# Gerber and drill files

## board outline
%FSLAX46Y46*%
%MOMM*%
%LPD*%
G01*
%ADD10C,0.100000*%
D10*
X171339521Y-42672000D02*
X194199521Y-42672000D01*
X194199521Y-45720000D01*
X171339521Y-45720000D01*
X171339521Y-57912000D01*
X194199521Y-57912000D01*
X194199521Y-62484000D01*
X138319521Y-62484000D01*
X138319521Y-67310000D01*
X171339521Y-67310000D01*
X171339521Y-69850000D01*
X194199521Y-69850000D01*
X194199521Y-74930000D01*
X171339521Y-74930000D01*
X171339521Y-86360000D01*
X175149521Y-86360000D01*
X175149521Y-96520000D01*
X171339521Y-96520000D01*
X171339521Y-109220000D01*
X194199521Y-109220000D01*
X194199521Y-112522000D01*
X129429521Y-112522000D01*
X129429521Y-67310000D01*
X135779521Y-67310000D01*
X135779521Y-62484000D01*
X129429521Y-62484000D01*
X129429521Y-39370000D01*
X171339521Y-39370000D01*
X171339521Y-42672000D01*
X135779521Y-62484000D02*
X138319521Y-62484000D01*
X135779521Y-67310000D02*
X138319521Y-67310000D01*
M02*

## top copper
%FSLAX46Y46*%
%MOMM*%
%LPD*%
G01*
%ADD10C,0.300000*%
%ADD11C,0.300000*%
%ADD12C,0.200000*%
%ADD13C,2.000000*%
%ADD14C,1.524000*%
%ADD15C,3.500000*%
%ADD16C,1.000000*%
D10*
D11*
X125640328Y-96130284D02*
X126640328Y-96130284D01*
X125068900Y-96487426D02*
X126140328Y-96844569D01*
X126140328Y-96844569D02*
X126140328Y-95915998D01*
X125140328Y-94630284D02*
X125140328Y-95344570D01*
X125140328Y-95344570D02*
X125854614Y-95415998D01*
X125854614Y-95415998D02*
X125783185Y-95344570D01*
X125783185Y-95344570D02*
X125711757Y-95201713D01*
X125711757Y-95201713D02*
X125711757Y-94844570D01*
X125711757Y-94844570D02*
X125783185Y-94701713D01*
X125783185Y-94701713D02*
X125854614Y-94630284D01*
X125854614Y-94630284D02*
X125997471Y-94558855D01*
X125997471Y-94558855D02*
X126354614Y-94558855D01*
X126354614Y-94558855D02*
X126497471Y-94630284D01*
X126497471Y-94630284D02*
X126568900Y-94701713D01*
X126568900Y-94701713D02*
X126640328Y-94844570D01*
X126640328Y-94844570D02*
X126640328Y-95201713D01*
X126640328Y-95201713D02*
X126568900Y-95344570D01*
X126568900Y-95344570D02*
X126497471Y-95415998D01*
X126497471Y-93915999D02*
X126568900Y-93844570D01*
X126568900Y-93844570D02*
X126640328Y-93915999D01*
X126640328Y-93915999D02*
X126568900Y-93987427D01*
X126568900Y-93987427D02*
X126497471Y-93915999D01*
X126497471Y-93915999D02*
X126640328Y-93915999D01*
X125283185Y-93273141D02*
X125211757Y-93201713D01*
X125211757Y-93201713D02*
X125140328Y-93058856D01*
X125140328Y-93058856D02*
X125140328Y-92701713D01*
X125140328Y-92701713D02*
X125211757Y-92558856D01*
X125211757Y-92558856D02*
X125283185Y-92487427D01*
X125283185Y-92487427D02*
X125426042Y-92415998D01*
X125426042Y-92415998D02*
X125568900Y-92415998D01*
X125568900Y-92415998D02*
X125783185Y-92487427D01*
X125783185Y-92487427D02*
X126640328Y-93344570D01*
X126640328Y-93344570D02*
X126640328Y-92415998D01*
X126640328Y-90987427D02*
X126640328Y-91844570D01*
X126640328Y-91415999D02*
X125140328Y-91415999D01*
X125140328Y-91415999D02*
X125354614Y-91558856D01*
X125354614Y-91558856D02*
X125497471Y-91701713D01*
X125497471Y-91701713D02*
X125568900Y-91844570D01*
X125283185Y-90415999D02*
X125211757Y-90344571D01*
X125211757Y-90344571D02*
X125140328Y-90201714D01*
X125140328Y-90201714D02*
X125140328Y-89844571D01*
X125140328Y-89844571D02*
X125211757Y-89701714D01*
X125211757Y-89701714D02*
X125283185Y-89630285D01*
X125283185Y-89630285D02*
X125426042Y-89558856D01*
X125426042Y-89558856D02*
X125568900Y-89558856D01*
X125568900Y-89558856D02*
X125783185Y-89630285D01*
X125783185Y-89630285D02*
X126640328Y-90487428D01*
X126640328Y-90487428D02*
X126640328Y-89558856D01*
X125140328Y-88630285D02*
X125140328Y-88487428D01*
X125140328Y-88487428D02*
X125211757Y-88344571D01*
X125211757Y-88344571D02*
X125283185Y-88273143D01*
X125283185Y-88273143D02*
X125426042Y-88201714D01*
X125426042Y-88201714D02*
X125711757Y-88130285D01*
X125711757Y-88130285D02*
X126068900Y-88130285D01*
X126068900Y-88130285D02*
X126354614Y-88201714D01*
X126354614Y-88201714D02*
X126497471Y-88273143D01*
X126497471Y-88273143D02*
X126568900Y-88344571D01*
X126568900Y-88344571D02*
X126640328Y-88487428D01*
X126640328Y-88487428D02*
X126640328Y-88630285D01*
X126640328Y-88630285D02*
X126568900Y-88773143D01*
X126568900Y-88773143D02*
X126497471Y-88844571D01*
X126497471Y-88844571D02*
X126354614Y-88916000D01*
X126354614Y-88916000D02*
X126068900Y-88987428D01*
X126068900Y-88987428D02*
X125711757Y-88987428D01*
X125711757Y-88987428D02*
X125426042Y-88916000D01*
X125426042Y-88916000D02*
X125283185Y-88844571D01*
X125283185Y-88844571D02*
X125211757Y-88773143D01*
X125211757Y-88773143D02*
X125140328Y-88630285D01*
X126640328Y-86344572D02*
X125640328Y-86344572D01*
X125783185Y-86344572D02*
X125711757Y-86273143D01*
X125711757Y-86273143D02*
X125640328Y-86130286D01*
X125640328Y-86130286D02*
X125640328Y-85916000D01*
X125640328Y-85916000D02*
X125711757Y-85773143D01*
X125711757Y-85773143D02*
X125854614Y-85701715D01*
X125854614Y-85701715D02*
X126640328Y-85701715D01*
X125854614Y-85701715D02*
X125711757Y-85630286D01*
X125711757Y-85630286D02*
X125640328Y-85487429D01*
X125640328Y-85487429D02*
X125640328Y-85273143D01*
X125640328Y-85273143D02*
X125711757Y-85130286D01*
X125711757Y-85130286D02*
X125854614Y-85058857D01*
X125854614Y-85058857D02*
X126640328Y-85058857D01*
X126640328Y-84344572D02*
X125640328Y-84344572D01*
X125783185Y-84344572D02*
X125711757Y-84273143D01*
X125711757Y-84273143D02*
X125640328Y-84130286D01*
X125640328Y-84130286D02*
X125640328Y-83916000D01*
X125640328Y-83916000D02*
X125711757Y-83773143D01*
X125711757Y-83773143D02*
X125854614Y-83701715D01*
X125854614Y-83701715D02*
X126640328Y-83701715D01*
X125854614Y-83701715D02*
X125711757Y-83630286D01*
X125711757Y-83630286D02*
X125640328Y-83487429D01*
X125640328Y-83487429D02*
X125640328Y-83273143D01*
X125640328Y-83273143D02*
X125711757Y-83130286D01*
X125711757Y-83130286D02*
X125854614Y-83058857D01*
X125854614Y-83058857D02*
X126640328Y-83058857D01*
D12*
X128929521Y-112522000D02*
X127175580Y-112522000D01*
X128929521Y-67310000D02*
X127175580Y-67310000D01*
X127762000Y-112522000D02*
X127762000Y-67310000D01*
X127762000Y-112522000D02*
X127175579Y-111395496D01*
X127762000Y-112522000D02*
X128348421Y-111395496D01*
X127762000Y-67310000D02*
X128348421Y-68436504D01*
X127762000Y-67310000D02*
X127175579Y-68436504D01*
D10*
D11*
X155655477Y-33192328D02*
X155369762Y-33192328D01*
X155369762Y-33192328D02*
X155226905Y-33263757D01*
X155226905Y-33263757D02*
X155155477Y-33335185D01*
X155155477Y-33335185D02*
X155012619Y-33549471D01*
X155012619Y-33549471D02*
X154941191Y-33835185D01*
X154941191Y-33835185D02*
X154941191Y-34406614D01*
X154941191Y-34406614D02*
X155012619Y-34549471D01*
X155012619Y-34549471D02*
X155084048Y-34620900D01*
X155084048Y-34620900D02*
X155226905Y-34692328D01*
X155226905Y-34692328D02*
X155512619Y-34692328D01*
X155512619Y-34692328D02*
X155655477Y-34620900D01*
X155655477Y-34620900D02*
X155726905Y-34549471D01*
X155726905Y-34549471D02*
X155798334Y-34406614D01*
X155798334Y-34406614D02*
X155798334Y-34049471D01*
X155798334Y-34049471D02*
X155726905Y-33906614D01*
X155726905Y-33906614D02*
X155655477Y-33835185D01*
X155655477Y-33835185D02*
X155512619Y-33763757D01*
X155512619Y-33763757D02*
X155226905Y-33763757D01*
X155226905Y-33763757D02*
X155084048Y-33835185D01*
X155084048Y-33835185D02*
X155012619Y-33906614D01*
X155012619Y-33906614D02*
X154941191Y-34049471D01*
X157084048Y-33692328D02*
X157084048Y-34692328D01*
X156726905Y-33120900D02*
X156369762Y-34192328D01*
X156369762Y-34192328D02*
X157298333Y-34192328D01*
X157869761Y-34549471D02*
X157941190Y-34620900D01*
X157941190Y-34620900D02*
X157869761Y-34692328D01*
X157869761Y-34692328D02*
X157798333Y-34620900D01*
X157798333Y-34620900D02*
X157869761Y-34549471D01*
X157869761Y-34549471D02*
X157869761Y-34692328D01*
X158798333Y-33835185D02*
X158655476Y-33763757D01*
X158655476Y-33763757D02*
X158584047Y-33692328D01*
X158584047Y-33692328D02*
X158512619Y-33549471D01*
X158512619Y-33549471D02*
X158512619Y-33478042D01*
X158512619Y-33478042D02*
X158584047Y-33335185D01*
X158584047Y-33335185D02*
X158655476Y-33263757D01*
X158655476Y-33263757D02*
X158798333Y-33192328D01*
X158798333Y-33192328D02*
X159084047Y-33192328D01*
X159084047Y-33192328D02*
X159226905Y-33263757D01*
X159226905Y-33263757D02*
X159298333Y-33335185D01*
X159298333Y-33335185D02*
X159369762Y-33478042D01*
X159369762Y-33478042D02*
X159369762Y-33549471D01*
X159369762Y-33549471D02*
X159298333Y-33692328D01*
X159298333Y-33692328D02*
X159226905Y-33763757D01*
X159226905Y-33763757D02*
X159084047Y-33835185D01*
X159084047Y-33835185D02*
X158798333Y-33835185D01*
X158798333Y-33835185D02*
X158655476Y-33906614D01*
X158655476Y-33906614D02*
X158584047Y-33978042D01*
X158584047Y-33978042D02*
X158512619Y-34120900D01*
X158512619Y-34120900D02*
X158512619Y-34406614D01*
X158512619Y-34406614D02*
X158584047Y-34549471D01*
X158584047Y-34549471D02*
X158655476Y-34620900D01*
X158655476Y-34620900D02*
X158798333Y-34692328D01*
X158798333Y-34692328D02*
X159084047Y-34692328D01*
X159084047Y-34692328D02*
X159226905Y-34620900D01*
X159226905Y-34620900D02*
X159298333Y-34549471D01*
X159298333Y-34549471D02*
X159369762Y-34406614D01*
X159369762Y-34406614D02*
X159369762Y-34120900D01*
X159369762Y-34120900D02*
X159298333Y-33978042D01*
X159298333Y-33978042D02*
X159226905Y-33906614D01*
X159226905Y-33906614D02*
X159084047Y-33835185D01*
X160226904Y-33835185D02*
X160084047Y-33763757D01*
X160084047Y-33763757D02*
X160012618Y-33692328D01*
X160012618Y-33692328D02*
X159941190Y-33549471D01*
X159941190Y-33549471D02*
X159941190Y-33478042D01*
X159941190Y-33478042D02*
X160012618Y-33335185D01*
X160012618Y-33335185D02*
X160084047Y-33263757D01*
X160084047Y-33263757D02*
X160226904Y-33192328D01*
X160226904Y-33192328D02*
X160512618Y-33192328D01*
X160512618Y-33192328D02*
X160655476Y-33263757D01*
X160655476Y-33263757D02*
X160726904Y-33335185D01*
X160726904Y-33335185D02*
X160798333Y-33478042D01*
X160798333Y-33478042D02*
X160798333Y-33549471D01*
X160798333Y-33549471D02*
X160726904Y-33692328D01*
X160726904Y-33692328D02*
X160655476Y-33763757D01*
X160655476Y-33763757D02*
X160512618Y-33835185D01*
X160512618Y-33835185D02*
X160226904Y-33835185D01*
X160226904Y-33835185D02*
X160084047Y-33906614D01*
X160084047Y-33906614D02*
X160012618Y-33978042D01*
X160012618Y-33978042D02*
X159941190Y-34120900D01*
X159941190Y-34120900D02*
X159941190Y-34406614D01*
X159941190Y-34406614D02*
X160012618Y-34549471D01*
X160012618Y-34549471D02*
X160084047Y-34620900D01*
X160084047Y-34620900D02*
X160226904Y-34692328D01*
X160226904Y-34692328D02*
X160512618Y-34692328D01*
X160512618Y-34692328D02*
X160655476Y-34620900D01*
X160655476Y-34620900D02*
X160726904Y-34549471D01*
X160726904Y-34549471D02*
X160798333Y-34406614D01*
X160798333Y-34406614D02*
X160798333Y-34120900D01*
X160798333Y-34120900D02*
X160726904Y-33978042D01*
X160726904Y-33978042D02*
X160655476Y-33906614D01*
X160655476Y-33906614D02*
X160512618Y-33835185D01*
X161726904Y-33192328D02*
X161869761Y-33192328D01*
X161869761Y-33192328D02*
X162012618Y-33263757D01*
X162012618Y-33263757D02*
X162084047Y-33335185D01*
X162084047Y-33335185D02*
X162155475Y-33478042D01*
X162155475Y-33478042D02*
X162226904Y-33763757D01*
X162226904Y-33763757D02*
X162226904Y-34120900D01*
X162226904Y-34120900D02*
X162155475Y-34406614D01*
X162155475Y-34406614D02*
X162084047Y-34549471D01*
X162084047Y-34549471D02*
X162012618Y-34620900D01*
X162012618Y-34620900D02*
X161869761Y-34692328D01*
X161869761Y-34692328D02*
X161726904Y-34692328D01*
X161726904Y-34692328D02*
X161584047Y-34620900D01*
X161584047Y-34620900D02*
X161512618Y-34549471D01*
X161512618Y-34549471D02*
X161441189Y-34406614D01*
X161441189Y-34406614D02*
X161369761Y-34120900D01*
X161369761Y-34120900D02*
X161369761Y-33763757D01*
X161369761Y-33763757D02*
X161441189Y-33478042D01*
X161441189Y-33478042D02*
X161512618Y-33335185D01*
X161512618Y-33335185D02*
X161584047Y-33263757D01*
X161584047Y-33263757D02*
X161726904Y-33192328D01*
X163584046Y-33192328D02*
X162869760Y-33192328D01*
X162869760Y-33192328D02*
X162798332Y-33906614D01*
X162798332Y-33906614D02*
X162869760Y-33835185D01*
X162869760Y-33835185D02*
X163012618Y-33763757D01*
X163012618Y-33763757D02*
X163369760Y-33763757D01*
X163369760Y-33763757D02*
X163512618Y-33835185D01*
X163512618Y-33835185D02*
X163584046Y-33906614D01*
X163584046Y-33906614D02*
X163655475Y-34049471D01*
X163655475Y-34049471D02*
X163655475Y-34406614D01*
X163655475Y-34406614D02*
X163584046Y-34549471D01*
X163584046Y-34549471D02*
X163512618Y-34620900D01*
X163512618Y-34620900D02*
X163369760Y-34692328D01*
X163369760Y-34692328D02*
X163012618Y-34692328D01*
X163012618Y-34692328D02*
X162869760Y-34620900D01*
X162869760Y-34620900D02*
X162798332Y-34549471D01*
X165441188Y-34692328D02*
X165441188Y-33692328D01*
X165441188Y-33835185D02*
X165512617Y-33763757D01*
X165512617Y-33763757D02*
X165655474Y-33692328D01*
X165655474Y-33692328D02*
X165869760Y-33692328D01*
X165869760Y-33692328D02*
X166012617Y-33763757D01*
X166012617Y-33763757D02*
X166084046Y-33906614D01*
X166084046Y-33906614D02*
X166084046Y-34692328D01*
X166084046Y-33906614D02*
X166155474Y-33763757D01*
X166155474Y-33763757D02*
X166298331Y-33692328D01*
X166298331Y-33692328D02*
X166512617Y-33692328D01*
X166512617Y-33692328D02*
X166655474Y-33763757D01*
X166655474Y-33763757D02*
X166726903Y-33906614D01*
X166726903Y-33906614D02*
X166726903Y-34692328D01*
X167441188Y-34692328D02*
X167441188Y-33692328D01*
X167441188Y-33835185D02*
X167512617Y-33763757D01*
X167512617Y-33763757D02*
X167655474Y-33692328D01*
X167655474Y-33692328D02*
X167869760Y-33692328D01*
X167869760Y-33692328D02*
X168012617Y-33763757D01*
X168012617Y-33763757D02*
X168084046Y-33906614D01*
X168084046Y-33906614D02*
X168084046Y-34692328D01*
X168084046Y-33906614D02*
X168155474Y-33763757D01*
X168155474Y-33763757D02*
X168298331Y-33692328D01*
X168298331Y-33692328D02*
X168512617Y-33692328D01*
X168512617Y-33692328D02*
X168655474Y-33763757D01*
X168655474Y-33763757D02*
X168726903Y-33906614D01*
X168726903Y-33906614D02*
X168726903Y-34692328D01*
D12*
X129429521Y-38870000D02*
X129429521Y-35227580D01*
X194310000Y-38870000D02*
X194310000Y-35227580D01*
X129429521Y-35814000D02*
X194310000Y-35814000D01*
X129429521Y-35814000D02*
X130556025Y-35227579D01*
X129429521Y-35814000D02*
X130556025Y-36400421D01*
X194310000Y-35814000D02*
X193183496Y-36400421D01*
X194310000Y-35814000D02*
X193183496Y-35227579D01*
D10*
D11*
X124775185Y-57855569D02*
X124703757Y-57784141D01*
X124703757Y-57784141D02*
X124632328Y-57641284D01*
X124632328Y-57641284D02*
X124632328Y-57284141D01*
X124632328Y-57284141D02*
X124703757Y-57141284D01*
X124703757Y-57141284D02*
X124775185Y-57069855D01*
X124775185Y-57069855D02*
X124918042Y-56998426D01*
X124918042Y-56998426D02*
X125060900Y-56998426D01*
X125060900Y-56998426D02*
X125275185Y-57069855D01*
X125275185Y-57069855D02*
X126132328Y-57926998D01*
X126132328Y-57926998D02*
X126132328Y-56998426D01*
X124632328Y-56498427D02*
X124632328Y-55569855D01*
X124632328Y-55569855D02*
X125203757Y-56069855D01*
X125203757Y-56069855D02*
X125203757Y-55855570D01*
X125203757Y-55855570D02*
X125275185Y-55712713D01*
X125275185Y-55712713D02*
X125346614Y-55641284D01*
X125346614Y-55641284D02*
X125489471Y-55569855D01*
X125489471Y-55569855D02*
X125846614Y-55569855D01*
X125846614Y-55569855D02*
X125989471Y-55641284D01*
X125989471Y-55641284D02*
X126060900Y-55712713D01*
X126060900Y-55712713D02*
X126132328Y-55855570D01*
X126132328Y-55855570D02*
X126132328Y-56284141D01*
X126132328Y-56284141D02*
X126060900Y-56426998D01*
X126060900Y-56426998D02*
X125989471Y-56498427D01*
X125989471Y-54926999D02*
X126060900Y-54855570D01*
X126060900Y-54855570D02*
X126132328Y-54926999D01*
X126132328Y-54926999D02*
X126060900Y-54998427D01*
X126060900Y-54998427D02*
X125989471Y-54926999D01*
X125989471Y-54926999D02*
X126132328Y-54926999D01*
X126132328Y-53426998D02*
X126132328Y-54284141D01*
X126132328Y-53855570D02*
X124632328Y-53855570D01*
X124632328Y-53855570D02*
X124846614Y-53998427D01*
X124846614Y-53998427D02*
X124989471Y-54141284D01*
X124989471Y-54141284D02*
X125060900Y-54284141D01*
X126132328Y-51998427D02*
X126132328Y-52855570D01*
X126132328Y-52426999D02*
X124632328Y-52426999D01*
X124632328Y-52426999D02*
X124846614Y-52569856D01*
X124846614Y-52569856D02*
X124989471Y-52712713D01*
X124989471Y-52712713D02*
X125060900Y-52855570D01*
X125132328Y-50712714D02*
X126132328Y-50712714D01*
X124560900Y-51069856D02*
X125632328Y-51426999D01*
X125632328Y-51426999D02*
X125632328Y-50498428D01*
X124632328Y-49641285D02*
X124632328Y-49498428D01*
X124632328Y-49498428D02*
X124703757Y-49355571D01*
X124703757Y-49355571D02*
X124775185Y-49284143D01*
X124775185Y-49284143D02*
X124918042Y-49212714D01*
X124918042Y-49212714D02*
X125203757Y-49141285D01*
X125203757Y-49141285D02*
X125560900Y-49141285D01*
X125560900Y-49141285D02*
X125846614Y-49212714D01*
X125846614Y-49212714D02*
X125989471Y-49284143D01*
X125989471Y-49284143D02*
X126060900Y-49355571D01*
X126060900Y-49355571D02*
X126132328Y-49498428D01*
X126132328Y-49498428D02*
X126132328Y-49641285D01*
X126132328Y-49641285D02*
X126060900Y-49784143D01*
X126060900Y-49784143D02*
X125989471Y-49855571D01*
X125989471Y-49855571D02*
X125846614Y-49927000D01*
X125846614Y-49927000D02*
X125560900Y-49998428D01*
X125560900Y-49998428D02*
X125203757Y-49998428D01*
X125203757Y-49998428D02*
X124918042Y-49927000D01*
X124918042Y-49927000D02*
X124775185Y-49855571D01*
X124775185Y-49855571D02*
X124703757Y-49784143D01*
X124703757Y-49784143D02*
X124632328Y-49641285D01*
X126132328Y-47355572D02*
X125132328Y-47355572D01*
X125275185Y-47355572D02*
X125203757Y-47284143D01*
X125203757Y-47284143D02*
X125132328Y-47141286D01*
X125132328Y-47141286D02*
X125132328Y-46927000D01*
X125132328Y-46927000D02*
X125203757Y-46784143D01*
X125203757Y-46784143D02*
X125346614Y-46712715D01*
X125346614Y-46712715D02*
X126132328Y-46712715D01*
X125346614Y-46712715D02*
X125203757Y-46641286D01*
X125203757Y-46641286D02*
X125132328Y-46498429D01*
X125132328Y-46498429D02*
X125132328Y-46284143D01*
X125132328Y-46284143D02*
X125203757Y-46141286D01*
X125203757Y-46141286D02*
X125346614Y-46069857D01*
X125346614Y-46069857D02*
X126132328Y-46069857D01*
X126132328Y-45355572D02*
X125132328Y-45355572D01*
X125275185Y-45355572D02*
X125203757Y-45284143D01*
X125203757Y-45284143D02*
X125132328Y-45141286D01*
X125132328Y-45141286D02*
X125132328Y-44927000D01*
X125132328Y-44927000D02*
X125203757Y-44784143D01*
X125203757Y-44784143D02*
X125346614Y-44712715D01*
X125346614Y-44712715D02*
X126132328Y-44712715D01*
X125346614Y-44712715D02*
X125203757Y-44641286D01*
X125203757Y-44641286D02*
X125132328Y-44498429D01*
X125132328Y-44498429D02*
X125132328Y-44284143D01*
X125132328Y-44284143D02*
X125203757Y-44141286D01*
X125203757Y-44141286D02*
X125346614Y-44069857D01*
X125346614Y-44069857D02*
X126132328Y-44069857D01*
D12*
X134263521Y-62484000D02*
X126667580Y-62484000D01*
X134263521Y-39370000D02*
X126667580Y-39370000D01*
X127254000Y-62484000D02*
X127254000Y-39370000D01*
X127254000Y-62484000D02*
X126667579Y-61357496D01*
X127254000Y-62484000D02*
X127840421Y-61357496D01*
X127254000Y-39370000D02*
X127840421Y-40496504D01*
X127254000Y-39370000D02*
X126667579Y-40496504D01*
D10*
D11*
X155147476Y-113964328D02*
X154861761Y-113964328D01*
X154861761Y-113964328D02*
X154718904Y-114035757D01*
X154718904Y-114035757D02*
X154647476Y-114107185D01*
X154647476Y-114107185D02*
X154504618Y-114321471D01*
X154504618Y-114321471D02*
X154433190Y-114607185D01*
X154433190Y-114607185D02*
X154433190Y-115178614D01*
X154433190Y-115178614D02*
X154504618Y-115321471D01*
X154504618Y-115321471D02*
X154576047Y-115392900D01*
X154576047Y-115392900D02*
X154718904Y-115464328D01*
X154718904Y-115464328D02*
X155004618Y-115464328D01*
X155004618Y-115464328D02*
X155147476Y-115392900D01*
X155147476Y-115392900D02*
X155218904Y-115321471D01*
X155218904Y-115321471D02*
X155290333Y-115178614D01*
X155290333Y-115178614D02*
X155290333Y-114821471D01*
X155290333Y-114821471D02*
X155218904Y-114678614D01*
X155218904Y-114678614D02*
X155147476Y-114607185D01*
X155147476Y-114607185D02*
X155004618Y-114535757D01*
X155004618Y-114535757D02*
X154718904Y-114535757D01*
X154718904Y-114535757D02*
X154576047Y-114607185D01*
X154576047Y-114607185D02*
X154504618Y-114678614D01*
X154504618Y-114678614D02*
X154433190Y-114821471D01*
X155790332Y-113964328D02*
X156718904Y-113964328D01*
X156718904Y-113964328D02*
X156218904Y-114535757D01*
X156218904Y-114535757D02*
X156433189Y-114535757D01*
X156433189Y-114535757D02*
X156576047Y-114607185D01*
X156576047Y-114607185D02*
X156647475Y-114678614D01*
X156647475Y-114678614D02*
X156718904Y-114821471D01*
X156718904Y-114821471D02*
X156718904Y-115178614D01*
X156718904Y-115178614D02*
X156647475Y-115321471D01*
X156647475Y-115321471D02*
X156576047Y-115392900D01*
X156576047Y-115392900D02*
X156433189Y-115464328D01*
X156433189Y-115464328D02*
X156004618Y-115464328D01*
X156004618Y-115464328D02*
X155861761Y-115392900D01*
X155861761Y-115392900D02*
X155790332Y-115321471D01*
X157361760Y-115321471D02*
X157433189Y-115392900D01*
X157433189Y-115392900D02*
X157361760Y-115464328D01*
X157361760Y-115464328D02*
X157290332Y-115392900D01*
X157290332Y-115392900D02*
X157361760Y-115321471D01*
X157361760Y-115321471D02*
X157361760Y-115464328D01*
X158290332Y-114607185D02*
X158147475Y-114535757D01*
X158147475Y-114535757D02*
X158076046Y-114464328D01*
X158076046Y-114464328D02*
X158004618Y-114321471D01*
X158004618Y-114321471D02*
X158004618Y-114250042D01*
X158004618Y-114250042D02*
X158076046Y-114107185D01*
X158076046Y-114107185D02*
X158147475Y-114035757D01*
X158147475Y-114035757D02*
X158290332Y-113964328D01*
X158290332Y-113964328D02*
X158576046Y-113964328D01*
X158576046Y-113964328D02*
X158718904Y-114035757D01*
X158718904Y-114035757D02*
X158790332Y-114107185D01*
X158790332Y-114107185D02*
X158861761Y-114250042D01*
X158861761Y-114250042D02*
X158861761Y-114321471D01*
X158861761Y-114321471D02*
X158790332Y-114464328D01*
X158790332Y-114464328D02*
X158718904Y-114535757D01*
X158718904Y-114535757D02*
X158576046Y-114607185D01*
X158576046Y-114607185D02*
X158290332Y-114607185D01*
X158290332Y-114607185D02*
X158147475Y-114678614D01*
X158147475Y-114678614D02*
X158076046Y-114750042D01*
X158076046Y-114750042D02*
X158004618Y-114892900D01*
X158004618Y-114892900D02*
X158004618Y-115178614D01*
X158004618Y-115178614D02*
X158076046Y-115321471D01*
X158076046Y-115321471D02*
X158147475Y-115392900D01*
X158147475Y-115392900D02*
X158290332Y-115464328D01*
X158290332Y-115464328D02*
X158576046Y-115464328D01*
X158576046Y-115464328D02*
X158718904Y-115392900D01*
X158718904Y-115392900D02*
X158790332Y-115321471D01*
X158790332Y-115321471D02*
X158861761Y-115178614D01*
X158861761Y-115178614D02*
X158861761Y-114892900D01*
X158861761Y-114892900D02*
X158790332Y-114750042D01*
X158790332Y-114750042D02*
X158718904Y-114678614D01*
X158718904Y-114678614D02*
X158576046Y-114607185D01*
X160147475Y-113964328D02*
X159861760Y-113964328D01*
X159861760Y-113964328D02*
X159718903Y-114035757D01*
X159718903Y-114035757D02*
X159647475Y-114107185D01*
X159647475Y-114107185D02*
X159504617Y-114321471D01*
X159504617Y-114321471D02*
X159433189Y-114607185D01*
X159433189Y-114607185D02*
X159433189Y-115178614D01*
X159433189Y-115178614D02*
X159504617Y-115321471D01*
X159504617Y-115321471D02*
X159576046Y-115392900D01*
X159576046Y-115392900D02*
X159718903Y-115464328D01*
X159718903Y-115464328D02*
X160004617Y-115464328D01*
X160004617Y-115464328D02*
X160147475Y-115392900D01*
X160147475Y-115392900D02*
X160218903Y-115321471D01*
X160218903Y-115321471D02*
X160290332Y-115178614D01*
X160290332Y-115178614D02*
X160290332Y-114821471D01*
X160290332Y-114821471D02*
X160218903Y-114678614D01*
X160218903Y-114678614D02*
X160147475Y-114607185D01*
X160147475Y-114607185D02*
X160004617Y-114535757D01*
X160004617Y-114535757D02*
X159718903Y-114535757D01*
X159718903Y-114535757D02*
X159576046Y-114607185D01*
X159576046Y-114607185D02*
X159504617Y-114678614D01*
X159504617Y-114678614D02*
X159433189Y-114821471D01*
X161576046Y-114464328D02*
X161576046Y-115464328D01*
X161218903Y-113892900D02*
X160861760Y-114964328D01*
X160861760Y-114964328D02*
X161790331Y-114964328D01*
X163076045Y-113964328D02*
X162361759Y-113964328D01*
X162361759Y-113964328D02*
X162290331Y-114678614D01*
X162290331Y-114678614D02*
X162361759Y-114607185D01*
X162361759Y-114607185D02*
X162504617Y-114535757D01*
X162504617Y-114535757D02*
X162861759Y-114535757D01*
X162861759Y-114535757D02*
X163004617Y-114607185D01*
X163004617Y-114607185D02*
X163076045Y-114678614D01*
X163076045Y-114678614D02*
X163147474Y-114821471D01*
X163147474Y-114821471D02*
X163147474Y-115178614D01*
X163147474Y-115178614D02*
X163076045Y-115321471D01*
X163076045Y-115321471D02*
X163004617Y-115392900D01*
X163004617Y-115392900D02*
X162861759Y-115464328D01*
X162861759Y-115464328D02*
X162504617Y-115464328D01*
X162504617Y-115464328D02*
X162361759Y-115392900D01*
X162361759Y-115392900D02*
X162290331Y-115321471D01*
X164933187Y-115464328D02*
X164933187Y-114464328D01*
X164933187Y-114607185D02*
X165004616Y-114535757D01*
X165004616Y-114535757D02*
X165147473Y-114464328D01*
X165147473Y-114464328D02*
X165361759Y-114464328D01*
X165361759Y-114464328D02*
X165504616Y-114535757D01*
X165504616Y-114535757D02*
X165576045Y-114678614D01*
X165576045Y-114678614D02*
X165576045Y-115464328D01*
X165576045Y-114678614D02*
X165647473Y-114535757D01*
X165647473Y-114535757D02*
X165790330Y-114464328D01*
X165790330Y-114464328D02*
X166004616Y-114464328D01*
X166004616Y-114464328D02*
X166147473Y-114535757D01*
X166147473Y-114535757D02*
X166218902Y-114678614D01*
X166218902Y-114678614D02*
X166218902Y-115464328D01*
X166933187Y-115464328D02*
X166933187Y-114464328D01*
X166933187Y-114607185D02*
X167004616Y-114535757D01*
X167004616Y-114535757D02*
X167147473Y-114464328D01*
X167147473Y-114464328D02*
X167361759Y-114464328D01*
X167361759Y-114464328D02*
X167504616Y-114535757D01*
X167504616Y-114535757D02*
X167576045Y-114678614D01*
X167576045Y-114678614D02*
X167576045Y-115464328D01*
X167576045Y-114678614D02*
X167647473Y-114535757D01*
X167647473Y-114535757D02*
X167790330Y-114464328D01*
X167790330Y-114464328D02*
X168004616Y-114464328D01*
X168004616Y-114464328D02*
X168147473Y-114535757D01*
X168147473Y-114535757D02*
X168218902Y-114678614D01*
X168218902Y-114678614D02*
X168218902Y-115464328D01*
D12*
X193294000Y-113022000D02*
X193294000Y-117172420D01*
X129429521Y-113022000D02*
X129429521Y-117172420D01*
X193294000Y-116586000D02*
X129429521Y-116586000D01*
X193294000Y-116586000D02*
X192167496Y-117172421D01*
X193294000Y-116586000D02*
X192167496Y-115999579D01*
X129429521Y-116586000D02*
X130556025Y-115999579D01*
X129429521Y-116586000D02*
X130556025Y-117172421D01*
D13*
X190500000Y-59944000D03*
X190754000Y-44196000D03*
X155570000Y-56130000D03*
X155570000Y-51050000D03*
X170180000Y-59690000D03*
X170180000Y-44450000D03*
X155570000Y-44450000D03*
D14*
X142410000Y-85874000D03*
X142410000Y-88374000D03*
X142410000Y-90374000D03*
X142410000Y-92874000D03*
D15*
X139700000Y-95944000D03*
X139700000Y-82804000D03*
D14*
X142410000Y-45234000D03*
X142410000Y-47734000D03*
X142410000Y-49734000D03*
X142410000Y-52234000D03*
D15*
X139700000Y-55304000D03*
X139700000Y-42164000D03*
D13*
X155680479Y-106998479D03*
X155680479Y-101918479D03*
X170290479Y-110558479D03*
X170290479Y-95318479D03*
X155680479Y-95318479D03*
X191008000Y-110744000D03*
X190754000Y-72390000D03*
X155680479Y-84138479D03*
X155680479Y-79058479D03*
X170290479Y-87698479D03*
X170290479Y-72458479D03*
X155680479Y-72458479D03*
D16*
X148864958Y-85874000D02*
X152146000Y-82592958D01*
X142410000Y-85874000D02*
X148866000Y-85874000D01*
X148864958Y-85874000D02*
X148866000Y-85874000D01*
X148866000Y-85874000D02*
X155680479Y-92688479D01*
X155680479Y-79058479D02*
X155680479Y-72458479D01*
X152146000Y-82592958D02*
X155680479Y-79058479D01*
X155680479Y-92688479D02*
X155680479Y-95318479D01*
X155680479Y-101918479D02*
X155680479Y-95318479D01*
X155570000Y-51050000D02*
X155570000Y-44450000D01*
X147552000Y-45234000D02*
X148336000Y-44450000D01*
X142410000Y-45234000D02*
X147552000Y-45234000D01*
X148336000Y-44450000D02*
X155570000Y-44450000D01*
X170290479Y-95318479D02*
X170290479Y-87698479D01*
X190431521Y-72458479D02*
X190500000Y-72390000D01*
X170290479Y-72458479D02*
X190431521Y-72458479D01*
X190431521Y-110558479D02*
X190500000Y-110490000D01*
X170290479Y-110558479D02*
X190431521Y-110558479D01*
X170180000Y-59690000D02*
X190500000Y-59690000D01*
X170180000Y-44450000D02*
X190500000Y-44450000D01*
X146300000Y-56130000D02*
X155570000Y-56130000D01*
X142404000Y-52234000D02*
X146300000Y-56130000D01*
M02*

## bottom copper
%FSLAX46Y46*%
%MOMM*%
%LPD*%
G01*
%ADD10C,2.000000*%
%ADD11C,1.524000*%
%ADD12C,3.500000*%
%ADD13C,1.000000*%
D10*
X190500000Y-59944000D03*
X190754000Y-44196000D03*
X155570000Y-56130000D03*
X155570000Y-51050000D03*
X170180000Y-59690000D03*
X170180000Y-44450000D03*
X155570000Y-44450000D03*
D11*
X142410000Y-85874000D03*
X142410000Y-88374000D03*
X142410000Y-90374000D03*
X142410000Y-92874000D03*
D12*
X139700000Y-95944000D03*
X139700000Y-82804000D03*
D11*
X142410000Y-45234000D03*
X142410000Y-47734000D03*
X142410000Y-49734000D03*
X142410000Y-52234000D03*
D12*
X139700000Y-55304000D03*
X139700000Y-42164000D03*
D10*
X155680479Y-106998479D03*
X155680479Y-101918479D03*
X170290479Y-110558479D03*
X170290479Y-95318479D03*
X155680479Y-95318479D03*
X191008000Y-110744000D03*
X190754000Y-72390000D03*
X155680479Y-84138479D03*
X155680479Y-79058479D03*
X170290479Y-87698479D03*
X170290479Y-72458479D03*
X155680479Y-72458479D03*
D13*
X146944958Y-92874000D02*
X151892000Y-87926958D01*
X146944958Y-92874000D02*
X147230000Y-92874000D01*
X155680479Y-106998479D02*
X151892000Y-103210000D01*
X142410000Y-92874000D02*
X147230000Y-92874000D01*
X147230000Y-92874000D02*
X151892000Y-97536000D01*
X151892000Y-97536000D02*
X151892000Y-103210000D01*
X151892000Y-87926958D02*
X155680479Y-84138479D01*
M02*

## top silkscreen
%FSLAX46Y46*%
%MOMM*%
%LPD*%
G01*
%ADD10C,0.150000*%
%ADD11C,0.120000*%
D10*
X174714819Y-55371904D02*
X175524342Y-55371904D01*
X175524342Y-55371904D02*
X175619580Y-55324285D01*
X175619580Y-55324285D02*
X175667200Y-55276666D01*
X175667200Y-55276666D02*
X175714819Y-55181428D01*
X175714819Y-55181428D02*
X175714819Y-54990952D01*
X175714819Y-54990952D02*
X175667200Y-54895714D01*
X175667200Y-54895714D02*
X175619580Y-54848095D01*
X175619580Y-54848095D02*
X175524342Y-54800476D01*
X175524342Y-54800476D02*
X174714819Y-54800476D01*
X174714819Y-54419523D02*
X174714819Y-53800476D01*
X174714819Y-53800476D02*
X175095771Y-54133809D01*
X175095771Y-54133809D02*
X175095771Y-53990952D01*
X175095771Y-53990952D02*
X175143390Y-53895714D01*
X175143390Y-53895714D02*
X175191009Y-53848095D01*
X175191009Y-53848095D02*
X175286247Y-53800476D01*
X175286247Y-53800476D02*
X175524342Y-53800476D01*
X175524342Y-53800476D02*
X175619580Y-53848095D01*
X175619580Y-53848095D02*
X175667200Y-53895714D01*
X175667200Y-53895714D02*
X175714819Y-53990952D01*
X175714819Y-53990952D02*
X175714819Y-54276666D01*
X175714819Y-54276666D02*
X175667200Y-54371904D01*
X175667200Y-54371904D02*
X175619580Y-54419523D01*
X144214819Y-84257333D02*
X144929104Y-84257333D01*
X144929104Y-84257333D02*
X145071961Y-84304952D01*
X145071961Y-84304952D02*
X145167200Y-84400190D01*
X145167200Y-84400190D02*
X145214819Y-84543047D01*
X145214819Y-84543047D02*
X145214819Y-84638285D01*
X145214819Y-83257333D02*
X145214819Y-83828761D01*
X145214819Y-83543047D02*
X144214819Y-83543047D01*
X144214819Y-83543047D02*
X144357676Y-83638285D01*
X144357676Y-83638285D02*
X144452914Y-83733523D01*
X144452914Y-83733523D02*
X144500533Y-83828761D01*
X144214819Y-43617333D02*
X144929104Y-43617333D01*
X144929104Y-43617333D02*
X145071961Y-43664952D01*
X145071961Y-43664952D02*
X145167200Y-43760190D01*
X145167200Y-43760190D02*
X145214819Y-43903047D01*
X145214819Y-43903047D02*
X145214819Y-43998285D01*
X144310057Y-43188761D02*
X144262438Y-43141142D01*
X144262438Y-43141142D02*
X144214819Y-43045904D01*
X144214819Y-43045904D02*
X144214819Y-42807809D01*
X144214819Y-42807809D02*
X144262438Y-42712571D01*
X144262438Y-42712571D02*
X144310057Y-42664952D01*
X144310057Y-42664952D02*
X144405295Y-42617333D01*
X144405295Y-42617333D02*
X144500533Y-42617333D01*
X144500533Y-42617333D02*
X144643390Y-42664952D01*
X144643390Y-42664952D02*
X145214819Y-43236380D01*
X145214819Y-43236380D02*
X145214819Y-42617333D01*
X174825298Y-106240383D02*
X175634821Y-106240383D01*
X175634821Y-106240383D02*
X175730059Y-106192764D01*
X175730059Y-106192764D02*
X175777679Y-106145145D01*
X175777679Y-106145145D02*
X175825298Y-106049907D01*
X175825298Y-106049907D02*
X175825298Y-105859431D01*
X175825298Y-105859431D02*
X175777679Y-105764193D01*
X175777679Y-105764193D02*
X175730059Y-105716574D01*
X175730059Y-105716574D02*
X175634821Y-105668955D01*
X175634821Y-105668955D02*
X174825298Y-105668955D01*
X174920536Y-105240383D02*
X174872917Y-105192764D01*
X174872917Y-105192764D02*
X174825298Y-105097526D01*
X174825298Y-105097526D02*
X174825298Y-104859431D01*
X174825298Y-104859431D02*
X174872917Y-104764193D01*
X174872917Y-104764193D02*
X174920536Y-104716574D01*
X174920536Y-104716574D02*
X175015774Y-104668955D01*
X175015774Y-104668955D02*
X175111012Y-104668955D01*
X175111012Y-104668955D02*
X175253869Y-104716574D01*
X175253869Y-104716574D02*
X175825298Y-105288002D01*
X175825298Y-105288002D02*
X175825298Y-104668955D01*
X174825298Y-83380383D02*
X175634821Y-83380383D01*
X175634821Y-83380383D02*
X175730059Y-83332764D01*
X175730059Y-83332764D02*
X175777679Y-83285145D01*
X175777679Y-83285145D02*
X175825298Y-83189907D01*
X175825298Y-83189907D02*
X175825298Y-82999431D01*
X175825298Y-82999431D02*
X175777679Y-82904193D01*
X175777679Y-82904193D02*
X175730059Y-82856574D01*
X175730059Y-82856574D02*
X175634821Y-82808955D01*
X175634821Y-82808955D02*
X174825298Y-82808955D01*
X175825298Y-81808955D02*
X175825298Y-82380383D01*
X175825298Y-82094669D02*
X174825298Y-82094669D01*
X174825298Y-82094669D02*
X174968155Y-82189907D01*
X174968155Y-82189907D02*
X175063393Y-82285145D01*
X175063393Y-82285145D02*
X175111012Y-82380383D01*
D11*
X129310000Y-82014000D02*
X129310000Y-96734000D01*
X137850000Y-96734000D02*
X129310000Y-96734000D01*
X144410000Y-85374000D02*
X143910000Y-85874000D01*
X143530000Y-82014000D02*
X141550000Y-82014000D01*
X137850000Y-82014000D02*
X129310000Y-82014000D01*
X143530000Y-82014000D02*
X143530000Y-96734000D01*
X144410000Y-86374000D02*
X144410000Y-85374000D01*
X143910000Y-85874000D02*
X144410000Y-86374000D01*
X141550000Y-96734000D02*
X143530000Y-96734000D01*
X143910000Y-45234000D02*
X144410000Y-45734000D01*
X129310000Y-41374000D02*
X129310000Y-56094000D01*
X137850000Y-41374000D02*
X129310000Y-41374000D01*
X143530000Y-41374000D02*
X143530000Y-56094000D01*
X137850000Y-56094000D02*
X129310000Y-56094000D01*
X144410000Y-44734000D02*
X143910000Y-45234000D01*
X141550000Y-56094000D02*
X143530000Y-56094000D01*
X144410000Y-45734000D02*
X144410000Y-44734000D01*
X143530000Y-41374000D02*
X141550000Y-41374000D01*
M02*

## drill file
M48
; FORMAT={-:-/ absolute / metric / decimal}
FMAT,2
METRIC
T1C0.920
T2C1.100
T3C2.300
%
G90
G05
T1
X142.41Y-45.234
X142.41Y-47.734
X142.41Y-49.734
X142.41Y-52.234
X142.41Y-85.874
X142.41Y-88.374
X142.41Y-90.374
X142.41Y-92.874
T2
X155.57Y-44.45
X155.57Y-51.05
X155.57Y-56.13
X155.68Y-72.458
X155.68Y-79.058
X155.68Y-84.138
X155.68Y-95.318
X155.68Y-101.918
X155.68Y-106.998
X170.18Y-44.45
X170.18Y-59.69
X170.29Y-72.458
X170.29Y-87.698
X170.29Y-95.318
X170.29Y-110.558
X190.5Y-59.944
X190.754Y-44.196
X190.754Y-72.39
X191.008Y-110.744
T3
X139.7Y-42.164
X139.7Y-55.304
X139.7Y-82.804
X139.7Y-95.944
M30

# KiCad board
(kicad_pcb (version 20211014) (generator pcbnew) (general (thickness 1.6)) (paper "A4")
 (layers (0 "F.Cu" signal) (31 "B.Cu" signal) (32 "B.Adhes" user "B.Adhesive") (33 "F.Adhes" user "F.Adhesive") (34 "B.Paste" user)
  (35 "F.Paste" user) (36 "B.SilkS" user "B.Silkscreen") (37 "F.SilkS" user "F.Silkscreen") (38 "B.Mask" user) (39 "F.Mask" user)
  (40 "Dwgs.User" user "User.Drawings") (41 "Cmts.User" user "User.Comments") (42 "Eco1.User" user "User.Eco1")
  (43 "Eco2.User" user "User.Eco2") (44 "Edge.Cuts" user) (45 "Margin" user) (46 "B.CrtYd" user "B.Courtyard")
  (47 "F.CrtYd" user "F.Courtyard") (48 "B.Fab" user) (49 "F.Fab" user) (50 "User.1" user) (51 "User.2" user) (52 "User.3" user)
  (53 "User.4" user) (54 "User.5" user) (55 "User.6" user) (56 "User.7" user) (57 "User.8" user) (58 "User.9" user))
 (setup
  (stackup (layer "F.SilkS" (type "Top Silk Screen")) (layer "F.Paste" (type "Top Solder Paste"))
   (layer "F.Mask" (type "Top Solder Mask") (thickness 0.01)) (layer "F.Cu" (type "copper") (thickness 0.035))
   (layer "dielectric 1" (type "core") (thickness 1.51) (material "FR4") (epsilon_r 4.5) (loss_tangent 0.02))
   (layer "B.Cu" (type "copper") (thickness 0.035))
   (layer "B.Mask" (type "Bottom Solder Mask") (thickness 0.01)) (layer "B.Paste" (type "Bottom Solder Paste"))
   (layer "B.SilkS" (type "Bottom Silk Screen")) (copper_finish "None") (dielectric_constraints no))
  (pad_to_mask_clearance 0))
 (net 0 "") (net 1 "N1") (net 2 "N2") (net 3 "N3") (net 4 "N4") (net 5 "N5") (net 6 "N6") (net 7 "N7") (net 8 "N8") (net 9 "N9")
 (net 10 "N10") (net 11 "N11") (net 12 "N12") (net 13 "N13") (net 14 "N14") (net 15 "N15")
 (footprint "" (layer "F.Cu") (at 190.5 59.944)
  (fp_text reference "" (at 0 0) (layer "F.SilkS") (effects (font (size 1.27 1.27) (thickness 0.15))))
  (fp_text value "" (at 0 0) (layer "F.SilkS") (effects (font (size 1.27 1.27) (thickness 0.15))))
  (pad "3" thru_hole circle (at 0 0 90) (size 2 2) (drill 1.1) (layers *.Cu *.Mask) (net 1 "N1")))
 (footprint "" (layer "F.Cu") (at 190.754 44.196)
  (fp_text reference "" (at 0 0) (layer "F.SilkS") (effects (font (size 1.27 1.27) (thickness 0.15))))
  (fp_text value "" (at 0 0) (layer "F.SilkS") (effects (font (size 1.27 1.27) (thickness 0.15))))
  (pad "4" thru_hole circle (at 0 0 90) (size 2 2) (drill 1.1) (layers *.Cu *.Mask) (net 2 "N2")))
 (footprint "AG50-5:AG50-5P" (layer "F.Cu") (at 170.18 54.61 90)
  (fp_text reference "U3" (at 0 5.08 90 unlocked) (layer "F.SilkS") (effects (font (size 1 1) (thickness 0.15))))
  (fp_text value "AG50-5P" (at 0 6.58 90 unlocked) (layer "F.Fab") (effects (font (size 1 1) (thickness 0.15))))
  (pad "1" thru_hole circle (at -1.52 -14.61 90) (size 2 2) (drill 1.1) (layers *.Cu *.Mask) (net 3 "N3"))
  (pad "2" thru_hole circle (at 3.56 -14.61 90) (size 2 2) (drill 1.1) (layers *.Cu *.Mask) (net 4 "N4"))
  (pad "3" thru_hole circle (at -5.08 0 90) (size 2 2) (drill 1.1) (layers *.Cu *.Mask) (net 1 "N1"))
  (pad "4" thru_hole circle (at 10.16 0 90) (size 2 2) (drill 1.1) (layers *.Cu *.Mask) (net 2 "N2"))
  (pad "5" thru_hole circle (at 10.16 -14.61 90) (size 2 2) (drill 1.1) (layers *.Cu *.Mask) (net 4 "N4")))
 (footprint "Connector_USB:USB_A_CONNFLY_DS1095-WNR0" (layer "F.Cu") (at 142.41 85.874 -90)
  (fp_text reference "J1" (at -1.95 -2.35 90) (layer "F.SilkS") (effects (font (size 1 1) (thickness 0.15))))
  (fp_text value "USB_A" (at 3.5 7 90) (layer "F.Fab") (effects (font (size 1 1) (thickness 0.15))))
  (fp_line (start -3.86 13.1) (end 10.86 13.1) (layer "F.SilkS") (width 0.12))
  (fp_line (start 10.86 4.56) (end 10.86 13.1) (layer "F.SilkS") (width 0.12))
  (fp_line (start -0.5 -2) (end 0 -1.5) (layer "F.SilkS") (width 0.12))
  (fp_line (start -3.86 -1.12) (end -3.86 0.86) (layer "F.SilkS") (width 0.12))
  (fp_line (start -3.86 4.56) (end -3.86 13.1) (layer "F.SilkS") (width 0.12))
  (fp_line (start -3.86 -1.12) (end 10.86 -1.12) (layer "F.SilkS") (width 0.12))
  (fp_line (start 0.5 -2) (end -0.5 -2) (layer "F.SilkS") (width 0.12))
  (fp_line (start 0 -1.5) (end 0.5 -2) (layer "F.SilkS") (width 0.12))
  (fp_line (start 10.86 0.86) (end 10.86 -1.12) (layer "F.SilkS") (width 0.12))
  (pad "1" thru_hole circle (at 0 0 270) (size 1.524 1.524) (drill 0.92) (layers *.Cu *.Mask) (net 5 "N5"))
  (pad "2" thru_hole circle (at 2.5 0 270) (size 1.524 1.524) (drill 0.92) (layers *.Cu *.Mask) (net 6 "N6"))
  (pad "3" thru_hole circle (at 4.5 0 270) (size 1.524 1.524) (drill 0.92) (layers *.Cu *.Mask) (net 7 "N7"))
  (pad "4" thru_hole circle (at 7 0 270) (size 1.524 1.524) (drill 0.92) (layers *.Cu *.Mask) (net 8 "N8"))
  (pad "5" thru_hole circle (at 10.07 2.71 270) (size 3.5 3.5) (drill 2.3) (layers *.Cu *.Mask) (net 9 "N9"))
  (pad "5" thru_hole circle (at -3.07 2.71 270) (size 3.5 3.5) (drill 2.3) (layers *.Cu *.Mask) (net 9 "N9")))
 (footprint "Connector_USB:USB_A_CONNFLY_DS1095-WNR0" (layer "F.Cu") (at 142.41 45.234 -90)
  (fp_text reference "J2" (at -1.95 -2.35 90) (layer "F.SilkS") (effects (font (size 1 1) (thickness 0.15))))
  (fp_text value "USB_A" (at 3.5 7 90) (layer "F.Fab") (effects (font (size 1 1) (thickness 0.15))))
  (fp_line (start 0 -1.5) (end 0.5 -2) (layer "F.SilkS") (width 0.12))
  (fp_line (start -3.86 13.1) (end 10.86 13.1) (layer "F.SilkS") (width 0.12))
  (fp_line (start -3.86 4.56) (end -3.86 13.1) (layer "F.SilkS") (width 0.12))
  (fp_line (start -3.86 -1.12) (end 10.86 -1.12) (layer "F.SilkS") (width 0.12))
  (fp_line (start 10.86 4.56) (end 10.86 13.1) (layer "F.SilkS") (width 0.12))
  (fp_line (start -0.5 -2) (end 0 -1.5) (layer "F.SilkS") (width 0.12))
  (fp_line (start 10.86 0.86) (end 10.86 -1.12) (layer "F.SilkS") (width 0.12))
  (fp_line (start 0.5 -2) (end -0.5 -2) (layer "F.SilkS") (width 0.12))
  (fp_line (start -3.86 -1.12) (end -3.86 0.86) (layer "F.SilkS") (width 0.12))
  (pad "1" thru_hole circle (at 0 0 270) (size 1.524 1.524) (drill 0.92) (layers *.Cu *.Mask) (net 4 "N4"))
  (pad "2" thru_hole circle (at 2.5 0 270) (size 1.524 1.524) (drill 0.92) (layers *.Cu *.Mask) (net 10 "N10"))
  (pad "3" thru_hole circle (at 4.5 0 270) (size 1.524 1.524) (drill 0.92) (layers *.Cu *.Mask) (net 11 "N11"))
  (pad "4" thru_hole circle (at 7 0 270) (size 1.524 1.524) (drill 0.92) (layers *.Cu *.Mask) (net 3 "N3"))
  (pad "5" thru_hole circle (at 10.07 2.71 270) (size 3.5 3.5) (drill 2.3) (layers *.Cu *.Mask) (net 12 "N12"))
  (pad "5" thru_hole circle (at -3.07 2.71 270) (size 3.5 3.5) (drill 2.3) (layers *.Cu *.Mask) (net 12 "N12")))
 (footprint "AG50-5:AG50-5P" (layer "F.Cu") (at 170.290479 105.478479 90)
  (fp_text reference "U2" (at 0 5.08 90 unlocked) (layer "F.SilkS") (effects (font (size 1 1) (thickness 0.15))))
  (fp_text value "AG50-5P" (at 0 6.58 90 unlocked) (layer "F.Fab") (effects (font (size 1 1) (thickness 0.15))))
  (pad "1" thru_hole circle (at -1.52 -14.61 90) (size 2 2) (drill 1.1) (layers *.Cu *.Mask) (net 8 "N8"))
  (pad "2" thru_hole circle (at 3.56 -14.61 90) (size 2 2) (drill 1.1) (layers *.Cu *.Mask) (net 5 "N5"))
  (pad "3" thru_hole circle (at -5.08 0 90) (size 2 2) (drill 1.1) (layers *.Cu *.Mask) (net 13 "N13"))
  (pad "4" thru_hole circle (at 10.16 0 90) (size 2 2) (drill 1.1) (layers *.Cu *.Mask) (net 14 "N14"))
  (pad "5" thru_hole circle (at 10.16 -14.61 90) (size 2 2) (drill 1.1) (layers *.Cu *.Mask) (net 5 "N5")))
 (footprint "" (layer "F.Cu") (at 191.008 110.744)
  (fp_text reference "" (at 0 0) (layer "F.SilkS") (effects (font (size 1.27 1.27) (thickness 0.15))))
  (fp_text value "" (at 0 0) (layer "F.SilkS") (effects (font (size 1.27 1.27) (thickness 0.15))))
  (pad "3" thru_hole circle (at 0 0 90) (size 2 2) (drill 1.1) (layers *.Cu *.Mask) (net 13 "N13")))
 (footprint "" (layer "F.Cu") (at 190.754 72.39)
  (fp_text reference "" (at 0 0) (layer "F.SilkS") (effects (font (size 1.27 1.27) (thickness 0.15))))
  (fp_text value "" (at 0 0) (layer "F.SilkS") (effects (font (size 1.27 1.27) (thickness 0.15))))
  (pad "4" thru_hole circle (at 0 0 90) (size 2 2) (drill 1.1) (layers *.Cu *.Mask) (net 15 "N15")))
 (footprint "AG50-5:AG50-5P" (layer "F.Cu") (at 170.290479 82.618479 90)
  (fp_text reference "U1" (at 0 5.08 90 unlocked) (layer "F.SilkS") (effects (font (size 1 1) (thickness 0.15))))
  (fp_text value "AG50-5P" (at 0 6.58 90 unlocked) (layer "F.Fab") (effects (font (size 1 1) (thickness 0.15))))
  (pad "1" thru_hole circle (at -1.52 -14.61 90) (size 2 2) (drill 1.1) (layers *.Cu *.Mask) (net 8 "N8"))
  (pad "2" thru_hole circle (at 3.56 -14.61 90) (size 2 2) (drill 1.1) (layers *.Cu *.Mask) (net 5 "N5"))
  (pad "3" thru_hole circle (at -5.08 0 90) (size 2 2) (drill 1.1) (layers *.Cu *.Mask) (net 14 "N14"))
  (pad "4" thru_hole circle (at 10.16 0 90) (size 2 2) (drill 1.1) (layers *.Cu *.Mask) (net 15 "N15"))
  (pad "5" thru_hole circle (at 10.16 -14.61 90) (size 2 2) (drill 1.1) (layers *.Cu *.Mask) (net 5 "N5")))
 (gr_poly
  (pts (xy 171.339521 42.672) (xy 194.199521 42.672) (xy 194.199521 45.72) (xy 171.339521 45.72) (xy 171.339521 57.912)
   (xy 194.199521 57.912) (xy 194.199521 62.484) (xy 138.319521 62.484) (xy 138.319521 67.31) (xy 171.339521 67.31) (xy 171.339521 69.85)
   (xy 194.199521 69.85) (xy 194.199521 74.93) (xy 171.339521 74.93) (xy 171.339521 86.36) (xy 175.149521 86.36) (xy 175.149521 96.52)
   (xy 171.339521 96.52) (xy 171.339521 109.22) (xy 194.199521 109.22) (xy 194.199521 112.522) (xy 129.429521 112.522) (xy 129.429521 67.31)
   (xy 135.779521 67.31) (xy 135.779521 62.484) (xy 129.429521 62.484) (xy 129.429521 39.37) (xy 171.339521 39.37))
  (layer "Edge.Cuts") (width 0.1) (fill none))
 (gr_line (start 135.779521 62.484) (end 138.319521 62.484) (layer "Edge.Cuts") (width 0.1))
 (gr_line (start 135.779521 67.31) (end 138.319521 67.31) (layer "Edge.Cuts") (width 0.1))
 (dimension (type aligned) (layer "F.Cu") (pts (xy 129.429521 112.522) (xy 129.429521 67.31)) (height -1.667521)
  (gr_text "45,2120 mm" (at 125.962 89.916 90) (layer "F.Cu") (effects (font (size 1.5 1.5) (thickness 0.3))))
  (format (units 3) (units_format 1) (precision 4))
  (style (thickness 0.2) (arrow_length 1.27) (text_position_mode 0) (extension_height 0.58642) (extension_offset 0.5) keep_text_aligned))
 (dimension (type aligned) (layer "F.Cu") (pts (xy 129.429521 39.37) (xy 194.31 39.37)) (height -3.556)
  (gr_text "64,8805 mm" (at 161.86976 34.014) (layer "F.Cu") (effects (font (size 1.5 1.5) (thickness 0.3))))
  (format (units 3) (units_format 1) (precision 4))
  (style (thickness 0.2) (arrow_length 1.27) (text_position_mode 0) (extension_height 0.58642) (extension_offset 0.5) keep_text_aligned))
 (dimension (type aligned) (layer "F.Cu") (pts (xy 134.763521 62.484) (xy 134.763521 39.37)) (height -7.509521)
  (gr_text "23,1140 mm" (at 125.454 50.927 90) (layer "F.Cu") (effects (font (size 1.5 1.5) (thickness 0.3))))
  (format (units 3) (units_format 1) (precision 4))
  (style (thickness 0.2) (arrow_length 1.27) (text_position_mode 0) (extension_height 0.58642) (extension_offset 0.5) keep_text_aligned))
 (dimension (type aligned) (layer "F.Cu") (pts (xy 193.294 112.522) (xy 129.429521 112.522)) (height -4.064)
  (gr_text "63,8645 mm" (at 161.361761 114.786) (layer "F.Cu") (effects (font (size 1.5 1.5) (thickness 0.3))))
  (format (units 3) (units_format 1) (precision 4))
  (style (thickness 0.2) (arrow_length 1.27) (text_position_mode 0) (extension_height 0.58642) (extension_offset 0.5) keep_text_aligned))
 (segment (start 148.864958 85.874) (end 152.146 82.592958) (width 1) (layer "F.Cu") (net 5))
 (segment (start 142.41 85.874) (end 148.866 85.874) (width 1) (layer "F.Cu") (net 5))
 (segment (start 148.864958 85.874) (end 148.866 85.874) (width 1) (layer "F.Cu") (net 5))
 (segment (start 148.866 85.874) (end 155.680479 92.688479) (width 1) (layer "F.Cu") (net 5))
 (segment (start 155.680479 79.058479) (end 155.680479 72.458479) (width 1) (layer "F.Cu") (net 5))
 (segment (start 152.146 82.592958) (end 155.680479 79.058479) (width 1) (layer "F.Cu") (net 5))
 (segment (start 155.680479 92.688479) (end 155.680479 95.318479) (width 1) (layer "F.Cu") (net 5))
 (segment (start 155.680479 101.918479) (end 155.680479 95.318479) (width 1) (layer "F.Cu") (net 5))
 (segment (start 155.57 51.05) (end 155.57 44.45) (width 1) (layer "F.Cu") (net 4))
 (segment (start 147.552 45.234) (end 148.336 44.45) (width 1) (layer "F.Cu") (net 4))
 (segment (start 142.41 45.234) (end 147.552 45.234) (width 1) (layer "F.Cu") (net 4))
 (segment (start 148.336 44.45) (end 155.57 44.45) (width 1) (layer "F.Cu") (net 4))
 (segment (start 146.944958 92.874) (end 151.892 87.926958) (width 1) (layer "B.Cu") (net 8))
 (segment (start 146.944958 92.874) (end 147.23 92.874) (width 1) (layer "B.Cu") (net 8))
 (segment (start 155.680479 106.998479) (end 151.892 103.21) (width 1) (layer "B.Cu") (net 8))
 (segment (start 142.41 92.874) (end 147.23 92.874) (width 1) (layer "B.Cu") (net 8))
 (segment (start 147.23 92.874) (end 151.892 97.536) (width 1) (layer "B.Cu") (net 8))
 (segment (start 151.892 97.536) (end 151.892 103.21) (width 1) (layer "B.Cu") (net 8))
 (segment (start 151.892 87.926958) (end 155.680479 84.138479) (width 1) (layer "B.Cu") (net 8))
 (segment (start 170.290479 95.318479) (end 170.290479 87.698479) (width 1) (layer "F.Cu") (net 14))
 (segment (start 190.431521 72.458479) (end 190.5 72.39) (width 1) (layer "F.Cu") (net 15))
 (segment (start 170.290479 72.458479) (end 190.431521 72.458479) (width 1) (layer "F.Cu") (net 15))
 (segment (start 190.431521 110.558479) (end 190.5 110.49) (width 1) (layer "F.Cu") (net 13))
 (segment (start 170.290479 110.558479) (end 190.431521 110.558479) (width 1) (layer "F.Cu") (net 13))
 (segment (start 170.18 59.69) (end 190.5 59.69) (width 1) (layer "F.Cu") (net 1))
 (segment (start 170.18 44.45) (end 190.5 44.45) (width 1) (layer "F.Cu") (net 2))
 (segment (start 146.3 56.13) (end 155.57 56.13) (width 1) (layer "F.Cu") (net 3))
 (segment (start 142.404 52.234) (end 146.3 56.13) (width 1) (layer "F.Cu") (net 3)))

